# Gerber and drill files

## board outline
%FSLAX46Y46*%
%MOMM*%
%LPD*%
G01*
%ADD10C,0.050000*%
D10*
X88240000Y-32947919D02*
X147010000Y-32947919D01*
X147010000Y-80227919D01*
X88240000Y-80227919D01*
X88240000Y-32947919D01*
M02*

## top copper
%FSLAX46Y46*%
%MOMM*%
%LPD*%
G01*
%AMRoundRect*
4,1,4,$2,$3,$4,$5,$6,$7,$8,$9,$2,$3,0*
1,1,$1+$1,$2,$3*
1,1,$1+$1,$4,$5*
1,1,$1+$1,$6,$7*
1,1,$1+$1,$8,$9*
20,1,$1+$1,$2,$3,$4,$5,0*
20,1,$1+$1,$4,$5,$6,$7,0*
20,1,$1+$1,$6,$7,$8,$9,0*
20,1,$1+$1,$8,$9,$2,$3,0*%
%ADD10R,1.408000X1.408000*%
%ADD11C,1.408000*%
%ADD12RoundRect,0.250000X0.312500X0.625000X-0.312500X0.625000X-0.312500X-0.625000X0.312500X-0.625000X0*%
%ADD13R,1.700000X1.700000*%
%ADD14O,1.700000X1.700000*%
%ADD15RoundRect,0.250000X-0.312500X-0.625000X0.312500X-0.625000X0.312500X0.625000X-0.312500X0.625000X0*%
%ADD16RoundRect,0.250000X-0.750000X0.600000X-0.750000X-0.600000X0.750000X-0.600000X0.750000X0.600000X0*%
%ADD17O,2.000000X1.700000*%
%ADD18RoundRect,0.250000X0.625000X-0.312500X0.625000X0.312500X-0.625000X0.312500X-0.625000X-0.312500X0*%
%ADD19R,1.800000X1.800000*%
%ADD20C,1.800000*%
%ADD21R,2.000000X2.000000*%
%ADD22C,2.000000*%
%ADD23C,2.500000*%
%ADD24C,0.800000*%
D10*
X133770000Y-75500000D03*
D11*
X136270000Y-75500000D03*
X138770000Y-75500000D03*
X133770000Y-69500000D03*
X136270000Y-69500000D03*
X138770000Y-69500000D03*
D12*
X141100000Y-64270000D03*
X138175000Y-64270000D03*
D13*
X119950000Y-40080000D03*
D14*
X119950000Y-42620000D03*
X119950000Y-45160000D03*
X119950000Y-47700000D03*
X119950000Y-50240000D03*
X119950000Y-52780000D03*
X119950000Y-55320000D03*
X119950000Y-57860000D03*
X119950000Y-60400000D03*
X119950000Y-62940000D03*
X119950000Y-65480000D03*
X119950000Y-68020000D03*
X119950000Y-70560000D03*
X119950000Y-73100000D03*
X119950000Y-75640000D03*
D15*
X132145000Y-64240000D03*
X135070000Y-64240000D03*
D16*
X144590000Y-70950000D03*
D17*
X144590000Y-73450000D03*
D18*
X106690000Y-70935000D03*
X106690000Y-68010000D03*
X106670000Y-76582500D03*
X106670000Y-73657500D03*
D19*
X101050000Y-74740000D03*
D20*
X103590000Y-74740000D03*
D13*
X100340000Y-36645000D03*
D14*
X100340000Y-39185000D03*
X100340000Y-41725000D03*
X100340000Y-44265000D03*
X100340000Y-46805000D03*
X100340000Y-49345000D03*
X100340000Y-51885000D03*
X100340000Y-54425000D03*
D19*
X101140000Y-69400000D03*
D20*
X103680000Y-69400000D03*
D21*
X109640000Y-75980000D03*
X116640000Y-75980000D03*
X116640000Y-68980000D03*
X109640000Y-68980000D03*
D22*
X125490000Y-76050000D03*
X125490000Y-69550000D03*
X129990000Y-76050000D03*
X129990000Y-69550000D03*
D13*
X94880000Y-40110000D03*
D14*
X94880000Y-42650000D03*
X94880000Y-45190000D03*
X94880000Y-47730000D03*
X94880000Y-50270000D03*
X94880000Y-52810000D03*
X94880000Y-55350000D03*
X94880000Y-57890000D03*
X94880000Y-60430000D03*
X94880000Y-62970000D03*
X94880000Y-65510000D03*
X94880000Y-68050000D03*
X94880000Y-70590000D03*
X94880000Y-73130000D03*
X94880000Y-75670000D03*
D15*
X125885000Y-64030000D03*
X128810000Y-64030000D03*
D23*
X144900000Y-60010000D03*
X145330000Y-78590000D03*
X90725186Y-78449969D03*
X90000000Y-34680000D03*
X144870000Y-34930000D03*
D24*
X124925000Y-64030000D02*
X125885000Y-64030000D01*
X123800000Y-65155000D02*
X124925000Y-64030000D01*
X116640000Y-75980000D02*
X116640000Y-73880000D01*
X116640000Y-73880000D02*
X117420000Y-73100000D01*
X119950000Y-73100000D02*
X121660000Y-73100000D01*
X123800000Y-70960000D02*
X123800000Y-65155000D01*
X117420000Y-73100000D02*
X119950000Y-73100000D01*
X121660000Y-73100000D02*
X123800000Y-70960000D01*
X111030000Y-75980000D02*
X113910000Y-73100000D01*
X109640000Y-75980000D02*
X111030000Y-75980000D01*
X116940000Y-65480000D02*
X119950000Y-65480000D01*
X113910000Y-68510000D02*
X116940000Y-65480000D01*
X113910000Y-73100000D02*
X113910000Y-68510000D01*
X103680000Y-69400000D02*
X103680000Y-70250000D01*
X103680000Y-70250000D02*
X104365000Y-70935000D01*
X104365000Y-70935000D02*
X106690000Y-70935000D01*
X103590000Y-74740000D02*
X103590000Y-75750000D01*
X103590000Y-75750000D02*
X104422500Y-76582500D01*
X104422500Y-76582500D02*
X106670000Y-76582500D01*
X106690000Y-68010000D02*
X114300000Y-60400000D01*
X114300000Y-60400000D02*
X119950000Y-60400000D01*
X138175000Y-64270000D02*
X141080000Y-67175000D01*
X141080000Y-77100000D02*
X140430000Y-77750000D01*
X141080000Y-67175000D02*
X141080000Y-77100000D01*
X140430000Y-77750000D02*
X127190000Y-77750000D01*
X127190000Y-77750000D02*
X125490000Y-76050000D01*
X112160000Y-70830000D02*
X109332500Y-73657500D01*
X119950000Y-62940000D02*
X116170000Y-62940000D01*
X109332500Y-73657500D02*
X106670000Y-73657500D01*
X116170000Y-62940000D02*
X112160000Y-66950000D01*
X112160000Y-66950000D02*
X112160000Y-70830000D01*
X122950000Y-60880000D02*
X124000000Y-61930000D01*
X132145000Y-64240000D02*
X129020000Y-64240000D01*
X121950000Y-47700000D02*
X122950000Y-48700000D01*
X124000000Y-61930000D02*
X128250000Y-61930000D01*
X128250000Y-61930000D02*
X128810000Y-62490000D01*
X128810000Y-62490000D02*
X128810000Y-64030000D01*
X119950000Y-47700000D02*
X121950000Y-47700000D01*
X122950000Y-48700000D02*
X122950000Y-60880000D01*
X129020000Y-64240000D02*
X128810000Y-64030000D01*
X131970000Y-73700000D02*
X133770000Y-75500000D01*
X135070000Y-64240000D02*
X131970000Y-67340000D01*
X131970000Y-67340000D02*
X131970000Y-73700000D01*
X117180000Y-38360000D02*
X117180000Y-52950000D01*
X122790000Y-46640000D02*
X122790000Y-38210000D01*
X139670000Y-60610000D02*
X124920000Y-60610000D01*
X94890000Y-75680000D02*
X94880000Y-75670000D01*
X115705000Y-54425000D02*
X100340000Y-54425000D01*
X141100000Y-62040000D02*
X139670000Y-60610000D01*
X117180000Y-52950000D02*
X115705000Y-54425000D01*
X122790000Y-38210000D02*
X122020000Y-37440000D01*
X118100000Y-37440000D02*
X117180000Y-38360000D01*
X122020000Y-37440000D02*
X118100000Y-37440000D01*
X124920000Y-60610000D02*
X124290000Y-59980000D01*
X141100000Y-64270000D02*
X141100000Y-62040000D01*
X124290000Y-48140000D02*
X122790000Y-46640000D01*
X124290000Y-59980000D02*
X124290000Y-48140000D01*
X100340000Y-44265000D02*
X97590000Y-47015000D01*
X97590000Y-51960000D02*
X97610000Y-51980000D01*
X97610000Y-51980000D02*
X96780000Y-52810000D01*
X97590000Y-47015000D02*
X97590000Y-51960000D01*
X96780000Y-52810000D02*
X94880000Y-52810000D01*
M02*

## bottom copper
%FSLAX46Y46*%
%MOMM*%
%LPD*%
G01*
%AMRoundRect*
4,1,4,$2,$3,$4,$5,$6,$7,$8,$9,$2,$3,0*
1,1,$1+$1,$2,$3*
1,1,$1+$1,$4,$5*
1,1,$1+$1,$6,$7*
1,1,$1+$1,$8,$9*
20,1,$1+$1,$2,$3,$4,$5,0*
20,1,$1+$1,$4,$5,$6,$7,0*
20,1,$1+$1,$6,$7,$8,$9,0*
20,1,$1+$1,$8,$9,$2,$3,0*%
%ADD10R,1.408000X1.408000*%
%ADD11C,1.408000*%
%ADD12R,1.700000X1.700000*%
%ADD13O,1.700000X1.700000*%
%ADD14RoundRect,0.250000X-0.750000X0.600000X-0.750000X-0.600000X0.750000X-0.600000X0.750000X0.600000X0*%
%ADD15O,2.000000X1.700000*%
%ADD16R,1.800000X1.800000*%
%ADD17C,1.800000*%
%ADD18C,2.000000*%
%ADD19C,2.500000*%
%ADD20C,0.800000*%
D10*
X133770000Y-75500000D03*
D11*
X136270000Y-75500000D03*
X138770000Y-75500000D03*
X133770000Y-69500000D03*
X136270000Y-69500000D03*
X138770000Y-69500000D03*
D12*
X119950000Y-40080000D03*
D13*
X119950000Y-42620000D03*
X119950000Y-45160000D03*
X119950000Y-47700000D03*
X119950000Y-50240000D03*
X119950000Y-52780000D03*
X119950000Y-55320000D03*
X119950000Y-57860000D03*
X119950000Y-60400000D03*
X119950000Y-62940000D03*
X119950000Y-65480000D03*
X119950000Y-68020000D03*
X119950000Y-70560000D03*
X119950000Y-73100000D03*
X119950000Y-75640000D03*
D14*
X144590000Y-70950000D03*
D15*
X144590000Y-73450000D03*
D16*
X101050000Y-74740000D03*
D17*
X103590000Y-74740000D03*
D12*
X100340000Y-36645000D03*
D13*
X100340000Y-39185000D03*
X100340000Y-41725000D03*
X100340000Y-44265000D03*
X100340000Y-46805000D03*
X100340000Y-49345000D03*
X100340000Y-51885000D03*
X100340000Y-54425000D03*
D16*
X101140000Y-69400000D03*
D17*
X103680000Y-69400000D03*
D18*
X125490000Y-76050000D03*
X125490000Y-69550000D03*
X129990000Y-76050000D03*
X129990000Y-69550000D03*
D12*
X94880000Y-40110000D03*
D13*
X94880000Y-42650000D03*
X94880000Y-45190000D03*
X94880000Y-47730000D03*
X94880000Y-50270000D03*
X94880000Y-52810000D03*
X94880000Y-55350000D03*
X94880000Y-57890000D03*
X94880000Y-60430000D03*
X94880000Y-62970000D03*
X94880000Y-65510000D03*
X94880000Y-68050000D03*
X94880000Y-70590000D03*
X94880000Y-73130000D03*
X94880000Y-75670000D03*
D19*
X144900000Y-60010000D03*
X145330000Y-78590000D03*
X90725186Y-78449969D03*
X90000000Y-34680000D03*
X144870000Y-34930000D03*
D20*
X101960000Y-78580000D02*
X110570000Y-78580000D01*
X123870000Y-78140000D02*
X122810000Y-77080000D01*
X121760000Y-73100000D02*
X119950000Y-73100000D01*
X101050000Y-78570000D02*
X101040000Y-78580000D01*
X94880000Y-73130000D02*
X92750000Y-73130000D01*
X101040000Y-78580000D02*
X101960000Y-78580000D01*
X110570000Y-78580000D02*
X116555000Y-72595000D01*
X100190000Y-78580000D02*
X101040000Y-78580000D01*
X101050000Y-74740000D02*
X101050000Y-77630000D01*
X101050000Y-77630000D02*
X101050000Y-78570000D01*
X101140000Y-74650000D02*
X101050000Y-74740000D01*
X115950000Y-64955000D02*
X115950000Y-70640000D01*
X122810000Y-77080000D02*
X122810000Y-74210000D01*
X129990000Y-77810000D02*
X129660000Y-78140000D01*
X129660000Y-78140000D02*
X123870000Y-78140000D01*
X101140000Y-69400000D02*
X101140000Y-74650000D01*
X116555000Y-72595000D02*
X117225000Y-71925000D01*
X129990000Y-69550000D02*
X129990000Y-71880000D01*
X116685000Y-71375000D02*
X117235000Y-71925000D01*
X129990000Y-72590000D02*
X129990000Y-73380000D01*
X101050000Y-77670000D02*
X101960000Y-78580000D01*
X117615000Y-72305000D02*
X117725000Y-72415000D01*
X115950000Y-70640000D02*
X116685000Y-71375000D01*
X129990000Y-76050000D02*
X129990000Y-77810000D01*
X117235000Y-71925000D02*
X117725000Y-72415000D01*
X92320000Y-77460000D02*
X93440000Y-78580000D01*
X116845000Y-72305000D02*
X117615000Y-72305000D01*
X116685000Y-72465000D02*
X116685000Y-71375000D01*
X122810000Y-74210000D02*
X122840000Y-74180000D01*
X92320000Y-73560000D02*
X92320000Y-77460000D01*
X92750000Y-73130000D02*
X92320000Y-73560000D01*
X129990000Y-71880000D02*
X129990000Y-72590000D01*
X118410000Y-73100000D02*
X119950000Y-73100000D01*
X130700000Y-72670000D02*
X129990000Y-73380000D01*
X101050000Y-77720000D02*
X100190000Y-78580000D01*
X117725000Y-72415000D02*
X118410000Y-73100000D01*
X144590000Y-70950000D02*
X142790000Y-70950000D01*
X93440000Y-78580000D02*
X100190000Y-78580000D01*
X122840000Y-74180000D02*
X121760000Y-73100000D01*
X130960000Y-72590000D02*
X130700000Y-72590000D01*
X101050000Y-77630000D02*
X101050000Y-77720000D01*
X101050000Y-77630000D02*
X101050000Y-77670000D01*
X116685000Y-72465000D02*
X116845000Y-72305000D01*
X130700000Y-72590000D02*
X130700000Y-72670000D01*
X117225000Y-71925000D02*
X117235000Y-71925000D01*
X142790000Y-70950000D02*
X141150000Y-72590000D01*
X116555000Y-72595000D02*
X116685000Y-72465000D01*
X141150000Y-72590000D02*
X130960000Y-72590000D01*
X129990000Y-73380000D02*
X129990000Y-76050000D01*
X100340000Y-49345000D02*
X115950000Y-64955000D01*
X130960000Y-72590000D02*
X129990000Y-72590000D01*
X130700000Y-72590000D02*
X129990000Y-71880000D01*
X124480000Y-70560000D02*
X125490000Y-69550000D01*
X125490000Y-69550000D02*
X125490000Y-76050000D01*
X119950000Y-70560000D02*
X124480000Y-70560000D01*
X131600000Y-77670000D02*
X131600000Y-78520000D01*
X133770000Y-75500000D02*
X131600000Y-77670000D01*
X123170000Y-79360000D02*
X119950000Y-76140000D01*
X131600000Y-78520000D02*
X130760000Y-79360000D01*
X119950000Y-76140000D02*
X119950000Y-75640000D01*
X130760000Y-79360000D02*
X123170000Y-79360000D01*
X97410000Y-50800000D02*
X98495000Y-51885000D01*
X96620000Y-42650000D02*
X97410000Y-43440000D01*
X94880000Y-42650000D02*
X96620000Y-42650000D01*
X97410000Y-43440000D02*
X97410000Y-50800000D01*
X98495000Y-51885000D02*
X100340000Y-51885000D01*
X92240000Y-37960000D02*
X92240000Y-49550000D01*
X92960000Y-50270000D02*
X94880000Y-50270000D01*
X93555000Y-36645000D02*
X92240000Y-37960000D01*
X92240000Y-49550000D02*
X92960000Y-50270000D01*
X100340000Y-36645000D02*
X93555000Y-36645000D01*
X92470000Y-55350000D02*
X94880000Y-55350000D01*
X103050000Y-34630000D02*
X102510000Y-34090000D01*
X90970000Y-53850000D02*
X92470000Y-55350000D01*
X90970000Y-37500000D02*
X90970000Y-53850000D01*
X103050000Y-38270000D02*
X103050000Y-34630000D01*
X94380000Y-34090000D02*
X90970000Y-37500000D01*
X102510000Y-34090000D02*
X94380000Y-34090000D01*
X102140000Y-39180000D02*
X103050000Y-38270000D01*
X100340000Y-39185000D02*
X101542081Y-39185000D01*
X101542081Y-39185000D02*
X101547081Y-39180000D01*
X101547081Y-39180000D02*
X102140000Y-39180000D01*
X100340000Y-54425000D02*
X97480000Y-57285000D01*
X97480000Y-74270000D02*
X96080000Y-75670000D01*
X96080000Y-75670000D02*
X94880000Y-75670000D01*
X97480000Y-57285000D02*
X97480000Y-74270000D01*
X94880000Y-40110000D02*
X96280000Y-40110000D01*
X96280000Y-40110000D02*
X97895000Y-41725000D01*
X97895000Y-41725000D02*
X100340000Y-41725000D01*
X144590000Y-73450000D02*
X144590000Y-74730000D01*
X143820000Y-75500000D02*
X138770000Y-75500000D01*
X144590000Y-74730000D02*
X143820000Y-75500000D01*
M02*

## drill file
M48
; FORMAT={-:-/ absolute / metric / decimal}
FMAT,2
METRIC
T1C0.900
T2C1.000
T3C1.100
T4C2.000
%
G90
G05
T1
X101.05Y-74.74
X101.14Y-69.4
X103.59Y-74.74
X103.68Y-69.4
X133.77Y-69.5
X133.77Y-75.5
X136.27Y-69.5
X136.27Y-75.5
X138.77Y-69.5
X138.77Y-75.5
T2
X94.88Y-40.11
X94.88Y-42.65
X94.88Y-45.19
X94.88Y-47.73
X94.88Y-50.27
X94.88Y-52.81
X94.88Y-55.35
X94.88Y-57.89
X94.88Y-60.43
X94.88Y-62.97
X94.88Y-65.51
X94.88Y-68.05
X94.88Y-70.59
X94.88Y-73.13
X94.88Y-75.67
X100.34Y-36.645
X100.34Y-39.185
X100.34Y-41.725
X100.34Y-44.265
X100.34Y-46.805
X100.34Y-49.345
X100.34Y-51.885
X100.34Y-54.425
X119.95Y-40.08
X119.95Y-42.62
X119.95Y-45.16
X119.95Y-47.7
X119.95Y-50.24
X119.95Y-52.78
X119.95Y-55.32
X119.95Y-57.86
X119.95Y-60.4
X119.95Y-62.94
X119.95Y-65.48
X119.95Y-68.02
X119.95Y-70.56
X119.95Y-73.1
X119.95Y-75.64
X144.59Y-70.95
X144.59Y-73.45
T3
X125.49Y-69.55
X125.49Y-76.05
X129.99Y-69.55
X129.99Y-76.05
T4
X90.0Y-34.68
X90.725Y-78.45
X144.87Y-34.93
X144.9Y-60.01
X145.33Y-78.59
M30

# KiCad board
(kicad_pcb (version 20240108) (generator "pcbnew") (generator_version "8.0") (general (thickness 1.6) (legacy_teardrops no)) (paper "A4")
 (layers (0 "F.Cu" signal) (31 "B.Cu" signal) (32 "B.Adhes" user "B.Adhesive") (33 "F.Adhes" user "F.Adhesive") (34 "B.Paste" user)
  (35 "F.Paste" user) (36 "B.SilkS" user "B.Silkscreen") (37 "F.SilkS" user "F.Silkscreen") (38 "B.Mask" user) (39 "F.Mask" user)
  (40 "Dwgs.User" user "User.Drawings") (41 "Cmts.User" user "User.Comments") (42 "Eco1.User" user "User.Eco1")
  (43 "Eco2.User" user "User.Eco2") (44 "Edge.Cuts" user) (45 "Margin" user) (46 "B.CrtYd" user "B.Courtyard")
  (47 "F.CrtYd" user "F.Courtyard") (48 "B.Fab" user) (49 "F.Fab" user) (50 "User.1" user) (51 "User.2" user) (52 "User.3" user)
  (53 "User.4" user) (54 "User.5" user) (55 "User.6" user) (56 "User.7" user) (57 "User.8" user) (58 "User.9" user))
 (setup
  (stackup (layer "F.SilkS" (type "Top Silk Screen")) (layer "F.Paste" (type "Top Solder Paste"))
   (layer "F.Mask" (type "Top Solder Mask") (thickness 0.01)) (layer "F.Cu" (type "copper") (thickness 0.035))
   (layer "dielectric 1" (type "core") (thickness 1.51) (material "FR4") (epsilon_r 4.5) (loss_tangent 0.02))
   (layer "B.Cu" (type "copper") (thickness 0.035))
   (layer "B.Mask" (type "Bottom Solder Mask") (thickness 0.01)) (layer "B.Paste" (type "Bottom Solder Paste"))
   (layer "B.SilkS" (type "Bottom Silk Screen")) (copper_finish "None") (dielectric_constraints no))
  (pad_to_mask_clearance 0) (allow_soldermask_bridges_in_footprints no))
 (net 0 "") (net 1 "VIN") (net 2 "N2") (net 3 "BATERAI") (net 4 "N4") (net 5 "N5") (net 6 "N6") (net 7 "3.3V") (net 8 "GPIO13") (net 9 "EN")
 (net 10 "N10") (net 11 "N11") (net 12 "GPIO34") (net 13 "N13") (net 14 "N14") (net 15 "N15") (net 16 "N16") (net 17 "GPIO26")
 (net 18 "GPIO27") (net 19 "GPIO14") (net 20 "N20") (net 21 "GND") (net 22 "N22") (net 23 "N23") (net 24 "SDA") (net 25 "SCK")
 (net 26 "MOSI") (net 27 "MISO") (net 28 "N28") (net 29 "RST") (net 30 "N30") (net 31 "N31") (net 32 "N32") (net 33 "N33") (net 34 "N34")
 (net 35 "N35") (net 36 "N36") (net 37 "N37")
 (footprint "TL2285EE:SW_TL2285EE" (layer "F.Cu") (at 136.27 72.5)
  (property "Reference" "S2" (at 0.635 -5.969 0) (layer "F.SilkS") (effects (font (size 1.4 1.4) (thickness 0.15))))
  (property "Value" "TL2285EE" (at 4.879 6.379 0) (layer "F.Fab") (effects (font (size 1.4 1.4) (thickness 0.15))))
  (pad "1" thru_hole rect (at -2.5 3) (size 1.408 1.408) (drill 0.9) (layers "*.Cu" "*.Mask") (remove_unused_layers no) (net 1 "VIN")
   (solder_mask_margin 0.102))
  (pad "2" thru_hole circle (at 0 3) (size 1.408 1.408) (drill 0.9) (layers "*.Cu" "*.Mask") (remove_unused_layers no) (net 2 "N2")
   (solder_mask_margin 0.102))
  (pad "3" thru_hole circle (at 2.5 3) (size 1.408 1.408) (drill 0.9) (layers "*.Cu" "*.Mask") (remove_unused_layers no) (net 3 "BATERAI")
   (solder_mask_margin 0.102))
  (pad "4" thru_hole circle (at -2.5 -3) (size 1.408 1.408) (drill 0.9) (layers "*.Cu" "*.Mask") (remove_unused_layers no) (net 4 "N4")
   (solder_mask_margin 0.102))
  (pad "5" thru_hole circle (at 0 -3) (size 1.408 1.408) (drill 0.9) (layers "*.Cu" "*.Mask") (remove_unused_layers no) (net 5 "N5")
   (solder_mask_margin 0.102))
  (pad "6" thru_hole circle (at 2.5 -3) (size 1.408 1.408) (drill 0.9) (layers "*.Cu" "*.Mask") (remove_unused_layers no) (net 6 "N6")
   (solder_mask_margin 0.102)))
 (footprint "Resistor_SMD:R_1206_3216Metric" (layer "F.Cu") (at 139.6375 64.27 180)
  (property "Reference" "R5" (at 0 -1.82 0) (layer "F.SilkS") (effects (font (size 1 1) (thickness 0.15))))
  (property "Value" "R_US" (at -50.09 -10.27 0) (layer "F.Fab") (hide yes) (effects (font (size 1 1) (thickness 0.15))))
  (pad "1" smd roundrect (at -1.4625 0 180) (size 1.125 1.75) (layers "F.Cu" "F.Paste" "F.Mask") (roundrect_rratio 0.222222) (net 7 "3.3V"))
  (pad "2" smd roundrect (at 1.4625 0 180) (size 1.125 1.75) (layers "F.Cu" "F.Paste" "F.Mask") (roundrect_rratio 0.222222) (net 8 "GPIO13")))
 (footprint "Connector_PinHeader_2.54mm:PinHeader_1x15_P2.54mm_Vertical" (layer "F.Cu") (at 119.95 40.08)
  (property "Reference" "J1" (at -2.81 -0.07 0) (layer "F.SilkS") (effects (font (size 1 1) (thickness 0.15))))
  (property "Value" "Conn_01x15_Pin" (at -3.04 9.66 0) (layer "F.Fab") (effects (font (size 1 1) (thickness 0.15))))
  (pad "1" thru_hole rect (at 0 0) (size 1.7 1.7) (drill 1) (layers "*.Cu" "*.Mask") (remove_unused_layers no) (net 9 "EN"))
  (pad "2" thru_hole oval (at 0 2.54) (size 1.7 1.7) (drill 1) (layers "*.Cu" "*.Mask") (remove_unused_layers no) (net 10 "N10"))
  (pad "3" thru_hole oval (at 0 5.08) (size 1.7 1.7) (drill 1) (layers "*.Cu" "*.Mask") (remove_unused_layers no) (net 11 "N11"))
  (pad "4" thru_hole oval (at 0 7.62) (size 1.7 1.7) (drill 1) (layers "*.Cu" "*.Mask") (remove_unused_layers no) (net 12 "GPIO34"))
  (pad "5" thru_hole oval (at 0 10.16) (size 1.7 1.7) (drill 1) (layers "*.Cu" "*.Mask") (remove_unused_layers no) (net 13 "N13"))
  (pad "6" thru_hole oval (at 0 12.7) (size 1.7 1.7) (drill 1) (layers "*.Cu" "*.Mask") (remove_unused_layers no) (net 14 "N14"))
  (pad "7" thru_hole oval (at 0 15.24) (size 1.7 1.7) (drill 1) (layers "*.Cu" "*.Mask") (remove_unused_layers no) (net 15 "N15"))
  (pad "8" thru_hole oval (at 0 17.78) (size 1.7 1.7) (drill 1) (layers "*.Cu" "*.Mask") (remove_unused_layers no) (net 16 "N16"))
  (pad "9" thru_hole oval (at 0 20.32) (size 1.7 1.7) (drill 1) (layers "*.Cu" "*.Mask") (remove_unused_layers no) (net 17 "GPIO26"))
  (pad "10" thru_hole oval (at 0 22.86) (size 1.7 1.7) (drill 1) (layers "*.Cu" "*.Mask") (remove_unused_layers no) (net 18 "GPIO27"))
  (pad "11" thru_hole oval (at 0 25.4) (size 1.7 1.7) (drill 1) (layers "*.Cu" "*.Mask") (remove_unused_layers no) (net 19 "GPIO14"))
  (pad "12" thru_hole oval (at 0 27.94) (size 1.7 1.7) (drill 1) (layers "*.Cu" "*.Mask") (remove_unused_layers no) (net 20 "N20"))
  (pad "13" thru_hole oval (at 0 30.48) (size 1.7 1.7) (drill 1) (layers "*.Cu" "*.Mask") (remove_unused_layers no) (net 8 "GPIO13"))
  (pad "14" thru_hole oval (at 0 33.02) (size 1.7 1.7) (drill 1) (layers "*.Cu" "*.Mask") (remove_unused_layers no) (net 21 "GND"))
  (pad "15" thru_hole oval (at 0 35.56) (size 1.7 1.7) (drill 1) (layers "*.Cu" "*.Mask") (remove_unused_layers no) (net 1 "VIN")))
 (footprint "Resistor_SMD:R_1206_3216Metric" (layer "F.Cu") (at 133.6075 64.24)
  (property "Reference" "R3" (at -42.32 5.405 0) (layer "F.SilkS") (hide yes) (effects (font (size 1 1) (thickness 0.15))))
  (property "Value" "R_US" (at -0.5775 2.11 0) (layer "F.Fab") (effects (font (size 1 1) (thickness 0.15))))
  (pad "1" smd roundrect (at -1.4625 0) (size 1.125 1.75) (layers "F.Cu" "F.Paste" "F.Mask") (roundrect_rratio 0.222222) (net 12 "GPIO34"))
  (pad "2" smd roundrect (at 1.4625 0) (size 1.125 1.75) (layers "F.Cu" "F.Paste" "F.Mask") (roundrect_rratio 0.222222) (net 1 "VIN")))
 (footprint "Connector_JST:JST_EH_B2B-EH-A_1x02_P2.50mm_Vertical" (layer "F.Cu") (at 144.59 70.95 -90)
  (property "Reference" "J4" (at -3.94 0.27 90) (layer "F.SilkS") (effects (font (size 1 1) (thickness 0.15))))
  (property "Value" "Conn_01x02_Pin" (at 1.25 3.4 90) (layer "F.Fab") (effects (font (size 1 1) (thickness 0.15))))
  (pad "1" thru_hole roundrect (at 0 0 270) (size 1.7 2) (drill 1) (layers "*.Cu" "*.Mask") (remove_unused_layers no)
   (roundrect_rratio 0.147059) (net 21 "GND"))
  (pad "2" thru_hole oval (at 2.5 0 270) (size 1.7 2) (drill 1) (layers "*.Cu" "*.Mask") (remove_unused_layers no) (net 3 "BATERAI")))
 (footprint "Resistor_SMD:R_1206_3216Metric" (layer "F.Cu") (at 106.69 69.4725 90)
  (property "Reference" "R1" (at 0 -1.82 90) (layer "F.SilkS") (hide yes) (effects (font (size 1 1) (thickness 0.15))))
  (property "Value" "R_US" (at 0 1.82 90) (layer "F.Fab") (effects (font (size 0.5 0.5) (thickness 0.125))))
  (pad "1" smd roundrect (at -1.4625 0 90) (size 1.125 1.75) (layers "F.Cu" "F.Paste" "F.Mask") (roundrect_rratio 0.222222) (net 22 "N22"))
  (pad "2" smd roundrect (at 1.4625 0 90) (size 1.125 1.75) (layers "F.Cu" "F.Paste" "F.Mask") (roundrect_rratio 0.222222) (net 17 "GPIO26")))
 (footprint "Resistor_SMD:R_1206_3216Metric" (layer "F.Cu") (at 106.67 75.12 90)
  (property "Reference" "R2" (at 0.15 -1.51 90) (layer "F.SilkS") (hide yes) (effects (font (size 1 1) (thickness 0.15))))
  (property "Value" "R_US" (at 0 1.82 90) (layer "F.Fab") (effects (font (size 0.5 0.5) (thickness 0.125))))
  (pad "1" smd roundrect (at -1.4625 0 90) (size 1.125 1.75) (layers "F.Cu" "F.Paste" "F.Mask") (roundrect_rratio 0.222222) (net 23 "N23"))
  (pad "2" smd roundrect (at 1.4625 0 90) (size 1.125 1.75) (layers "F.Cu" "F.Paste" "F.Mask") (roundrect_rratio 0.222222) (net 18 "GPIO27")))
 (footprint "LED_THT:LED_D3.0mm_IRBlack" (layer "F.Cu") (at 101.05 74.74)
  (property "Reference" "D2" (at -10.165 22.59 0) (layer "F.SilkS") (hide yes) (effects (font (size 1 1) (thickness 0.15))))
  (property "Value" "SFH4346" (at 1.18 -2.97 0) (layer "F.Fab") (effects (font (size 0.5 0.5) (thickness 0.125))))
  (pad "1" thru_hole rect (at 0 0) (size 1.8 1.8) (drill 0.9) (layers "*.Cu" "*.Mask") (remove_unused_layers no) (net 21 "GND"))
  (pad "2" thru_hole circle (at 2.54 0) (size 1.8 1.8) (drill 0.9) (layers "*.Cu" "*.Mask") (remove_unused_layers no) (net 23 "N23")))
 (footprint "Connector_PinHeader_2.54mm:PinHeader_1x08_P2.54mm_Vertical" (layer "F.Cu") (at 100.34 36.645)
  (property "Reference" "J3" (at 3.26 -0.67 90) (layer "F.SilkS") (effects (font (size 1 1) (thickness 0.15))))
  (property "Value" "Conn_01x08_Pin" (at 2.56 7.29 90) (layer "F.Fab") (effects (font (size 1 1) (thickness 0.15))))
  (pad "1" thru_hole rect (at 0 0) (size 1.7 1.7) (drill 1) (layers "*.Cu" "*.Mask") (remove_unused_layers no) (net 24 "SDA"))
  (pad "2" thru_hole oval (at 0 2.54) (size 1.7 1.7) (drill 1) (layers "*.Cu" "*.Mask") (remove_unused_layers no) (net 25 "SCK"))
  (pad "3" thru_hole oval (at 0 5.08) (size 1.7 1.7) (drill 1) (layers "*.Cu" "*.Mask") (remove_unused_layers no) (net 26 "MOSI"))
  (pad "4" thru_hole oval (at 0 7.62) (size 1.7 1.7) (drill 1) (layers "*.Cu" "*.Mask") (remove_unused_layers no) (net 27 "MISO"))
  (pad "5" thru_hole oval (at 0 10.16) (size 1.7 1.7) (drill 1) (layers "*.Cu" "*.Mask") (remove_unused_layers no) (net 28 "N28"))
  (pad "6" thru_hole oval (at 0 12.7) (size 1.7 1.7) (drill 1) (layers "*.Cu" "*.Mask") (remove_unused_layers no) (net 21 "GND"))
  (pad "7" thru_hole oval (at 0 15.24) (size 1.7 1.7) (drill 1) (layers "*.Cu" "*.Mask") (remove_unused_layers no) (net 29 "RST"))
  (pad "8" thru_hole oval (at 0 17.78) (size 1.7 1.7) (drill 1) (layers "*.Cu" "*.Mask") (remove_unused_layers no) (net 7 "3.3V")))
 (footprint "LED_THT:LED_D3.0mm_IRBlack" (layer "F.Cu") (at 101.14 69.4)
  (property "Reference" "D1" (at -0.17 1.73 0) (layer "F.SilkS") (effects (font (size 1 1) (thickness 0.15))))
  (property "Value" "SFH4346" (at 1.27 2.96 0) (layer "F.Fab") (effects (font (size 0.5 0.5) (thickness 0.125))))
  (pad "1" thru_hole rect (at 0 0) (size 1.8 1.8) (drill 0.9) (layers "*.Cu" "*.Mask") (remove_unused_layers no) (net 21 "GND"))
  (pad "2" thru_hole circle (at 2.54 0) (size 1.8 1.8) (drill 0.9) (layers "*.Cu" "*.Mask") (remove_unused_layers no) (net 22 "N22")))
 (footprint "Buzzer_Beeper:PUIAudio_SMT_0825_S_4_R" (layer "F.Cu") (at 113.14 72.48 90)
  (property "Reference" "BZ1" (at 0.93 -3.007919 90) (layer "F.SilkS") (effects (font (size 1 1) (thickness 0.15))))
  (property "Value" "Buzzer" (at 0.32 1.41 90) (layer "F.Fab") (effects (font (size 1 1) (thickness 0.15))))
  (pad "1" smd rect (at -3.5 -3.5) (size 2 2) (layers "F.Cu" "F.Paste" "F.Mask") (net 19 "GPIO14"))
  (pad "2" smd rect (at -3.5 3.5) (size 2 2) (layers "F.Cu" "F.Paste" "F.Mask") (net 21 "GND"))
  (pad "3" smd rect (at 3.5 3.5) (size 2 2) (layers "F.Cu" "F.Paste" "F.Mask"))
  (pad "4" smd rect (at 3.5 -3.5) (size 2 2) (layers "F.Cu" "F.Paste" "F.Mask")))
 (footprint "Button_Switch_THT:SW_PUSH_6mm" (layer "F.Cu") (at 125.49 76.05 90)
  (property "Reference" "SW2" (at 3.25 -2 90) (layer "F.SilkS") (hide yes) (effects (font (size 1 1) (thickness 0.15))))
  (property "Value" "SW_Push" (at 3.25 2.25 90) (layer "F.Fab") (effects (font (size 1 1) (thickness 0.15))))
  (pad "1" thru_hole circle (at 0 0 180) (size 2 2) (drill 1.1) (layers "*.Cu" "*.Mask") (remove_unused_layers no) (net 8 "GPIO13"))
  (pad "1" thru_hole circle (at 6.5 0 180) (size 2 2) (drill 1.1) (layers "*.Cu" "*.Mask") (remove_unused_layers no) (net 8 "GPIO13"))
  (pad "2" thru_hole circle (at 0 4.5 180) (size 2 2) (drill 1.1) (layers "*.Cu" "*.Mask") (remove_unused_layers no) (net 21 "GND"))
  (pad "2" thru_hole circle (at 6.5 4.5 180) (size 2 2) (drill 1.1) (layers "*.Cu" "*.Mask") (remove_unused_layers no) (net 21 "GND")))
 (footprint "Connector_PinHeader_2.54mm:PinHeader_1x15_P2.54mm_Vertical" (layer "F.Cu") (at 94.88 40.11)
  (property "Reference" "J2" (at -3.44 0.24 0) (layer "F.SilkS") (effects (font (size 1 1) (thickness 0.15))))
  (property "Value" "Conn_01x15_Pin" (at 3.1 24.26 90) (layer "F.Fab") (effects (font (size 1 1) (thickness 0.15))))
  (pad "1" thru_hole rect (at 0 0) (size 1.7 1.7) (drill 1) (layers "*.Cu" "*.Mask") (remove_unused_layers no) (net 26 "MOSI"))
  (pad "2" thru_hole oval (at 0 2.54) (size 1.7 1.7) (drill 1) (layers "*.Cu" "*.Mask") (remove_unused_layers no) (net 29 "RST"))
  (pad "3" thru_hole oval (at 0 5.08) (size 1.7 1.7) (drill 1) (layers "*.Cu" "*.Mask") (remove_unused_layers no) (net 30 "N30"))
  (pad "4" thru_hole oval (at 0 7.62) (size 1.7 1.7) (drill 1) (layers "*.Cu" "*.Mask") (remove_unused_layers no) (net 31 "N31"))
  (pad "5" thru_hole oval (at 0 10.16) (size 1.7 1.7) (drill 1) (layers "*.Cu" "*.Mask") (remove_unused_layers no) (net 24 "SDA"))
  (pad "6" thru_hole oval (at 0 12.7) (size 1.7 1.7) (drill 1) (layers "*.Cu" "*.Mask") (remove_unused_layers no) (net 27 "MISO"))
  (pad "7" thru_hole oval (at 0 15.24) (size 1.7 1.7) (drill 1) (layers "*.Cu" "*.Mask") (remove_unused_layers no) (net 25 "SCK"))
  (pad "8" thru_hole oval (at 0 17.78) (size 1.7 1.7) (drill 1) (layers "*.Cu" "*.Mask") (remove_unused_layers no) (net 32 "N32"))
  (pad "9" thru_hole oval (at 0 20.32) (size 1.7 1.7) (drill 1) (layers "*.Cu" "*.Mask") (remove_unused_layers no) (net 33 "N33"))
  (pad "10" thru_hole oval (at 0 22.86) (size 1.7 1.7) (drill 1) (layers "*.Cu" "*.Mask") (remove_unused_layers no) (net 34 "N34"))
  (pad "11" thru_hole oval (at 0 25.4) (size 1.7 1.7) (drill 1) (layers "*.Cu" "*.Mask") (remove_unused_layers no) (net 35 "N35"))
  (pad "12" thru_hole oval (at 0 27.94) (size 1.7 1.7) (drill 1) (layers "*.Cu" "*.Mask") (remove_unused_layers no) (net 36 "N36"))
  (pad "13" thru_hole oval (at 0 30.48) (size 1.7 1.7) (drill 1) (layers "*.Cu" "*.Mask") (remove_unused_layers no) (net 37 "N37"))
  (pad "14" thru_hole oval (at 0 33.02) (size 1.7 1.7) (drill 1) (layers "*.Cu" "*.Mask") (remove_unused_layers no) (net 21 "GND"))
  (pad "15" thru_hole oval (at 0 35.56) (size 1.7 1.7) (drill 1) (layers "*.Cu" "*.Mask") (remove_unused_layers no) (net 7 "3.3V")))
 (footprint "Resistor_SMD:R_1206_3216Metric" (layer "F.Cu") (at 127.3475 64.03)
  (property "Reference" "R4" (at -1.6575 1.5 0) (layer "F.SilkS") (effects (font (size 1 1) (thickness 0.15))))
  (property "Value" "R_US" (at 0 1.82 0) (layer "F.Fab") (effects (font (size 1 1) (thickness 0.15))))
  (pad "1" smd roundrect (at -1.4625 0) (size 1.125 1.75) (layers "F.Cu" "F.Paste" "F.Mask") (roundrect_rratio 0.222222) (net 21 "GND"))
  (pad "2" smd roundrect (at 1.4625 0) (size 1.125 1.75) (layers "F.Cu" "F.Paste" "F.Mask") (roundrect_rratio 0.222222) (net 12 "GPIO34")))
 (gr_rect (start 88.24 32.947919) (end 147.01 80.227919) (stroke (width 0.05) (type default)) (fill none) (layer "Edge.Cuts"))
 (via (at 144.9 60.01) (size 2.5) (drill 2) (layers "F.Cu" "B.Cu") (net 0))
 (via (at 145.33 78.59) (size 2.5) (drill 2) (layers "F.Cu" "B.Cu") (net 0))
 (via (at 90.725186 78.449969) (size 2.5) (drill 2) (layers "F.Cu" "B.Cu") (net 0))
 (via (at 90 34.68) (size 2.5) (drill 2) (layers "F.Cu" "B.Cu") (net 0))
 (via (at 144.87 34.93) (size 2.5) (drill 2) (layers "F.Cu" "B.Cu") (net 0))
 (segment (start 124.925 64.03) (end 125.885 64.03) (width 0.8) (layer "F.Cu") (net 21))
 (segment (start 123.8 65.155) (end 124.925 64.03) (width 0.8) (layer "F.Cu") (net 21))
 (segment (start 116.64 75.98) (end 116.64 73.88) (width 0.8) (layer "F.Cu") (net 21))
 (segment (start 116.64 73.88) (end 117.42 73.1) (width 0.8) (layer "F.Cu") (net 21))
 (segment (start 119.95 73.1) (end 121.66 73.1) (width 0.8) (layer "F.Cu") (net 21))
 (segment (start 123.8 70.96) (end 123.8 65.155) (width 0.8) (layer "F.Cu") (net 21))
 (segment (start 117.42 73.1) (end 119.95 73.1) (width 0.8) (layer "F.Cu") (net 21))
 (segment (start 121.66 73.1) (end 123.8 70.96) (width 0.8) (layer "F.Cu") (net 21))
 (segment (start 101.96 78.58) (end 110.57 78.58) (width 0.8) (layer "B.Cu") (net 21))
 (segment (start 123.87 78.14) (end 122.81 77.08) (width 0.8) (layer "B.Cu") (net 21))
 (segment (start 121.76 73.1) (end 119.95 73.1) (width 0.8) (layer "B.Cu") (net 21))
 (segment (start 101.05 78.57) (end 101.04 78.58) (width 0.8) (layer "B.Cu") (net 21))
 (segment (start 94.88 73.13) (end 92.75 73.13) (width 0.8) (layer "B.Cu") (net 21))
 (segment (start 101.04 78.58) (end 101.96 78.58) (width 0.8) (layer "B.Cu") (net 21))
 (segment (start 110.57 78.58) (end 116.555 72.595) (width 0.8) (layer "B.Cu") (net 21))
 (segment (start 100.19 78.58) (end 101.04 78.58) (width 0.8) (layer "B.Cu") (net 21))
 (segment (start 101.05 74.74) (end 101.05 77.63) (width 0.8) (layer "B.Cu") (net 21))
 (segment (start 101.05 77.63) (end 101.05 78.57) (width 0.8) (layer "B.Cu") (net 21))
 (segment (start 101.14 74.65) (end 101.05 74.74) (width 0.8) (layer "B.Cu") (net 21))
 (segment (start 115.95 64.955) (end 115.95 70.64) (width 0.8) (layer "B.Cu") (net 21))
 (segment (start 122.81 77.08) (end 122.81 74.21) (width 0.8) (layer "B.Cu") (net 21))
 (segment (start 129.99 77.81) (end 129.66 78.14) (width 0.8) (layer "B.Cu") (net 21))
 (segment (start 129.66 78.14) (end 123.87 78.14) (width 0.8) (layer "B.Cu") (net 21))
 (segment (start 101.14 69.4) (end 101.14 74.65) (width 0.8) (layer "B.Cu") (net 21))
 (segment (start 116.555 72.595) (end 117.225 71.925) (width 0.8) (layer "B.Cu") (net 21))
 (segment (start 129.99 69.55) (end 129.99 71.88) (width 0.8) (layer "B.Cu") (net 21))
 (segment (start 116.685 71.375) (end 117.235 71.925) (width 0.8) (layer "B.Cu") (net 21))
 (segment (start 129.99 72.59) (end 129.99 73.38) (width 0.8) (layer "B.Cu") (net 21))
 (segment (start 101.05 77.67) (end 101.96 78.58) (width 0.8) (layer "B.Cu") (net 21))
 (segment (start 117.615 72.305) (end 117.725 72.415) (width 0.8) (layer "B.Cu") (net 21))
 (segment (start 115.95 70.64) (end 116.685 71.375) (width 0.8) (layer "B.Cu") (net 21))
 (segment (start 129.99 76.05) (end 129.99 77.81) (width 0.8) (layer "B.Cu") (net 21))
 (segment (start 117.235 71.925) (end 117.725 72.415) (width 0.8) (layer "B.Cu") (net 21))
 (segment (start 92.32 77.46) (end 93.44 78.58) (width 0.8) (layer "B.Cu") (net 21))
 (segment (start 116.845 72.305) (end 117.615 72.305) (width 0.8) (layer "B.Cu") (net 21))
 (segment (start 116.685 72.465) (end 116.685 71.375) (width 0.8) (layer "B.Cu") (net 21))
 (segment (start 122.81 74.21) (end 122.84 74.18) (width 0.8) (layer "B.Cu") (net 21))
 (segment (start 92.32 73.56) (end 92.32 77.46) (width 0.8) (layer "B.Cu") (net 21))
 (segment (start 92.75 73.13) (end 92.32 73.56) (width 0.8) (layer "B.Cu") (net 21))
 (segment (start 129.99 71.88) (end 129.99 72.59) (width 0.8) (layer "B.Cu") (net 21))
 (segment (start 118.41 73.1) (end 119.95 73.1) (width 0.8) (layer "B.Cu") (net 21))
 (segment (start 130.7 72.67) (end 129.99 73.38) (width 0.8) (layer "B.Cu") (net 21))
 (segment (start 101.05 77.72) (end 100.19 78.58) (width 0.8) (layer "B.Cu") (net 21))
 (segment (start 117.725 72.415) (end 118.41 73.1) (width 0.8) (layer "B.Cu") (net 21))
 (segment (start 144.59 70.95) (end 142.79 70.95) (width 0.8) (layer "B.Cu") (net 21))
 (segment (start 93.44 78.58) (end 100.19 78.58) (width 0.8) (layer "B.Cu") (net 21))
 (segment (start 122.84 74.18) (end 121.76 73.1) (width 0.8) (layer "B.Cu") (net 21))
 (segment (start 130.96 72.59) (end 130.7 72.59) (width 0.8) (layer "B.Cu") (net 21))
 (segment (start 101.05 77.63) (end 101.05 77.72) (width 0.8) (layer "B.Cu") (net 21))
 (segment (start 101.05 77.63) (end 101.05 77.67) (width 0.8) (layer "B.Cu") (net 21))
 (segment (start 116.685 72.465) (end 116.845 72.305) (width 0.8) (layer "B.Cu") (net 21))
 (segment (start 130.7 72.59) (end 130.7 72.67) (width 0.8) (layer "B.Cu") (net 21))
 (segment (start 117.225 71.925) (end 117.235 71.925) (width 0.8) (layer "B.Cu") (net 21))
 (segment (start 142.79 70.95) (end 141.15 72.59) (width 0.8) (layer "B.Cu") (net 21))
 (segment (start 116.555 72.595) (end 116.685 72.465) (width 0.8) (layer "B.Cu") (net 21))
 (segment (start 141.15 72.59) (end 130.96 72.59) (width 0.8) (layer "B.Cu") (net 21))
 (segment (start 129.99 73.38) (end 129.99 76.05) (width 0.8) (layer "B.Cu") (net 21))
 (segment (start 100.34 49.345) (end 115.95 64.955) (width 0.8) (layer "B.Cu") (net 21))
 (segment (start 130.96 72.59) (end 129.99 72.59) (width 0.8) (layer "B.Cu") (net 21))
 (segment (start 130.7 72.59) (end 129.99 71.88) (width 0.8) (layer "B.Cu") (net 21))
 (segment (start 111.03 75.98) (end 113.91 73.1) (width 0.8) (layer "F.Cu") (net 19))
 (segment (start 109.64 75.98) (end 111.03 75.98) (width 0.8) (layer "F.Cu") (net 19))
 (segment (start 116.94 65.48) (end 119.95 65.48) (width 0.8) (layer "F.Cu") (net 19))
 (segment (start 113.91 68.51) (end 116.94 65.48) (width 0.8) (layer "F.Cu") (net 19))
 (segment (start 113.91 73.1) (end 113.91 68.51) (width 0.8) (layer "F.Cu") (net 19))
 (segment (start 103.68 69.4) (end 103.68 70.25) (width 0.8) (layer "F.Cu") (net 22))
 (segment (start 103.68 70.25) (end 104.365 70.935) (width 0.8) (layer "F.Cu") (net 22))
 (segment (start 104.365 70.935) (end 106.69 70.935) (width 0.8) (layer "F.Cu") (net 22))
 (segment (start 103.59 74.74) (end 103.59 75.75) (width 0.8) (layer "F.Cu") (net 23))
 (segment (start 103.59 75.75) (end 104.4225 76.5825) (width 0.8) (layer "F.Cu") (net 23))
 (segment (start 104.4225 76.5825) (end 106.67 76.5825) (width 0.8) (layer "F.Cu") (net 23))
 (segment (start 106.69 68.01) (end 114.3 60.4) (width 0.8) (layer "F.Cu") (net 17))
 (segment (start 114.3 60.4) (end 119.95 60.4) (width 0.8) (layer "F.Cu") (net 17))
 (segment (start 138.175 64.27) (end 141.08 67.175) (width 0.8) (layer "F.Cu") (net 8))
 (segment (start 141.08 77.1) (end 140.43 77.75) (width 0.8) (layer "F.Cu") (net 8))
 (segment (start 141.08 67.175) (end 141.08 77.1) (width 0.8) (layer "F.Cu") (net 8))
 (segment (start 140.43 77.75) (end 127.19 77.75) (width 0.8) (layer "F.Cu") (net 8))
 (segment (start 127.19 77.75) (end 125.49 76.05) (width 0.8) (layer "F.Cu") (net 8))
 (segment (start 124.48 70.56) (end 125.49 69.55) (width 0.8) (layer "B.Cu") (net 8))
 (segment (start 125.49 69.55) (end 125.49 76.05) (width 0.8) (layer "B.Cu") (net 8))
 (segment (start 119.95 70.56) (end 124.48 70.56) (width 0.8) (layer "B.Cu") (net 8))
 (segment (start 112.16 70.83) (end 109.3325 73.6575) (width 0.8) (layer "F.Cu") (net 18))
 (segment (start 119.95 62.94) (end 116.17 62.94) (width 0.8) (layer "F.Cu") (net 18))
 (segment (start 109.3325 73.6575) (end 106.67 73.6575) (width 0.8) (layer "F.Cu") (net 18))
 (segment (start 116.17 62.94) (end 112.16 66.95) (width 0.8) (layer "F.Cu") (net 18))
 (segment (start 112.16 66.95) (end 112.16 70.83) (width 0.8) (layer "F.Cu") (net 18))
 (segment (start 122.95 60.88) (end 124 61.93) (width 0.8) (layer "F.Cu") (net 12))
 (segment (start 132.145 64.24) (end 129.02 64.24) (width 0.8) (layer "F.Cu") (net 12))
 (segment (start 121.95 47.7) (end 122.95 48.7) (width 0.8) (layer "F.Cu") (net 12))
 (segment (start 124 61.93) (end 128.25 61.93) (width 0.8) (layer "F.Cu") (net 12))
 (segment (start 128.25 61.93) (end 128.81 62.49) (width 0.8) (layer "F.Cu") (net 12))
 (segment (start 128.81 62.49) (end 128.81 64.03) (width 0.8) (layer "F.Cu") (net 12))
 (segment (start 119.95 47.7) (end 121.95 47.7) (width 0.8) (layer "F.Cu") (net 12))
 (segment (start 122.95 48.7) (end 122.95 60.88) (width 0.8) (layer "F.Cu") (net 12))
 (segment (start 129.02 64.24) (end 128.81 64.03) (width 0.8) (layer "F.Cu") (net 12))
 (segment (start 131.97 73.7) (end 133.77 75.5) (width 0.8) (layer "F.Cu") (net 1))
 (segment (start 135.07 64.24) (end 131.97 67.34) (width 0.8) (layer "F.Cu") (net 1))
 (segment (start 131.97 67.34) (end 131.97 73.7) (width 0.8) (layer "F.Cu") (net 1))
 (segment (start 131.6 77.67) (end 131.6 78.52) (width 0.8) (layer "B.Cu") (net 1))
 (segment (start 133.77 75.5) (end 131.6 77.67) (width 0.8) (layer "B.Cu") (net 1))
 (segment (start 123.17 79.36) (end 119.95 76.14) (width 0.8) (layer "B.Cu") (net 1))
 (segment (start 131.6 78.52) (end 130.76 79.36) (width 0.8) (layer "B.Cu") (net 1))
 (segment (start 119.95 76.14) (end 119.95 75.64) (width 0.8) (layer "B.Cu") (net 1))
 (segment (start 130.76 79.36) (end 123.17 79.36) (width 0.8) (layer "B.Cu") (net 1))
 (segment (start 97.41 50.8) (end 98.495 51.885) (width 0.8) (layer "B.Cu") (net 29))
 (segment (start 96.62 42.65) (end 97.41 43.44) (width 0.8) (layer "B.Cu") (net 29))
 (segment (start 94.88 42.65) (end 96.62 42.65) (width 0.8) (layer "B.Cu") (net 29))
 (segment (start 97.41 43.44) (end 97.41 50.8) (width 0.8) (layer "B.Cu") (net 29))
 (segment (start 98.495 51.885) (end 100.34 51.885) (width 0.8) (layer "B.Cu") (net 29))
 (segment (start 92.24 37.96) (end 92.24 49.55) (width 0.8) (layer "B.Cu") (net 24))
 (segment (start 92.96 50.27) (end 94.88 50.27) (width 0.8) (layer "B.Cu") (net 24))
 (segment (start 93.555 36.645) (end 92.24 37.96) (width 0.8) (layer "B.Cu") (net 24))
 (segment (start 92.24 49.55) (end 92.96 50.27) (width 0.8) (layer "B.Cu") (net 24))
 (segment (start 100.34 36.645) (end 93.555 36.645) (width 0.8) (layer "B.Cu") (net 24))
 (segment (start 92.47 55.35) (end 94.88 55.35) (width 0.8) (layer "B.Cu") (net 25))
 (segment (start 103.05 34.63) (end 102.51 34.09) (width 0.8) (layer "B.Cu") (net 25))
 (segment (start 90.97 53.85) (end 92.47 55.35) (width 0.8) (layer "B.Cu") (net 25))
 (segment (start 90.97 37.5) (end 90.97 53.85) (width 0.8) (layer "B.Cu") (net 25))
 (segment (start 103.05 38.27) (end 103.05 34.63) (width 0.8) (layer "B.Cu") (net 25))
 (segment (start 94.38 34.09) (end 90.97 37.5) (width 0.8) (layer "B.Cu") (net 25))
 (segment (start 102.51 34.09) (end 94.38 34.09) (width 0.8) (layer "B.Cu") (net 25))
 (segment (start 102.14 39.18) (end 103.05 38.27) (width 0.8) (layer "B.Cu") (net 25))
 (segment (start 100.34 39.185) (end 101.542081 39.185) (width 0.8) (layer "B.Cu") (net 25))
 (segment (start 101.542081 39.185) (end 101.547081 39.18) (width 0.8) (layer "B.Cu") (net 25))
 (segment (start 101.547081 39.18) (end 102.14 39.18) (width 0.8) (layer "B.Cu") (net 25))
 (segment (start 117.18 38.36) (end 117.18 52.95) (width 0.8) (layer "F.Cu") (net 7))
 (segment (start 122.79 46.64) (end 122.79 38.21) (width 0.8) (layer "F.Cu") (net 7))
 (segment (start 139.67 60.61) (end 124.92 60.61) (width 0.8) (layer "F.Cu") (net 7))
 (segment (start 94.89 75.68) (end 94.88 75.67) (width 0.8) (layer "F.Cu") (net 7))
 (segment (start 115.705 54.425) (end 100.34 54.425) (width 0.8) (layer "F.Cu") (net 7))
 (segment (start 141.1 62.04) (end 139.67 60.61) (width 0.8) (layer "F.Cu") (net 7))
 (segment (start 117.18 52.95) (end 115.705 54.425) (width 0.8) (layer "F.Cu") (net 7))
 (segment (start 122.79 38.21) (end 122.02 37.44) (width 0.8) (layer "F.Cu") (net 7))
 (segment (start 118.1 37.44) (end 117.18 38.36) (width 0.8) (layer "F.Cu") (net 7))
 (segment (start 122.02 37.44) (end 118.1 37.44) (width 0.8) (layer "F.Cu") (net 7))
 (segment (start 124.92 60.61) (end 124.29 59.98) (width 0.8) (layer "F.Cu") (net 7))
 (segment (start 141.1 64.27) (end 141.1 62.04) (width 0.8) (layer "F.Cu") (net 7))
 (segment (start 124.29 48.14) (end 122.79 46.64) (width 0.8) (layer "F.Cu") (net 7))
 (segment (start 124.29 59.98) (end 124.29 48.14) (width 0.8) (layer "F.Cu") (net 7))
 (segment (start 100.34 54.425) (end 97.48 57.285) (width 0.8) (layer "B.Cu") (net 7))
 (segment (start 97.48 74.27) (end 96.08 75.67) (width 0.8) (layer "B.Cu") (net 7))
 (segment (start 96.08 75.67) (end 94.88 75.67) (width 0.8) (layer "B.Cu") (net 7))
 (segment (start 97.48 57.285) (end 97.48 74.27) (width 0.8) (layer "B.Cu") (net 7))
 (segment (start 94.88 40.11) (end 96.28 40.11) (width 0.8) (layer "B.Cu") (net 26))
 (segment (start 96.28 40.11) (end 97.895 41.725) (width 0.8) (layer "B.Cu") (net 26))
 (segment (start 97.895 41.725) (end 100.34 41.725) (width 0.8) (layer "B.Cu") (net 26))
 (segment (start 100.34 44.265) (end 97.59 47.015) (width 0.8) (layer "F.Cu") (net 27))
 (segment (start 97.59 51.96) (end 97.61 51.98) (width 0.8) (layer "F.Cu") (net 27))
 (segment (start 97.61 51.98) (end 96.78 52.81) (width 0.8) (layer "F.Cu") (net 27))
 (segment (start 97.59 47.015) (end 97.59 51.96) (width 0.8) (layer "F.Cu") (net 27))
 (segment (start 96.78 52.81) (end 94.88 52.81) (width 0.8) (layer "F.Cu") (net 27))
 (segment (start 144.59 73.45) (end 144.59 74.73) (width 0.8) (layer "B.Cu") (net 3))
 (segment (start 143.82 75.5) (end 138.77 75.5) (width 0.8) (layer "B.Cu") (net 3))
 (segment (start 144.59 74.73) (end 143.82 75.5) (width 0.8) (layer "B.Cu") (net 3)))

